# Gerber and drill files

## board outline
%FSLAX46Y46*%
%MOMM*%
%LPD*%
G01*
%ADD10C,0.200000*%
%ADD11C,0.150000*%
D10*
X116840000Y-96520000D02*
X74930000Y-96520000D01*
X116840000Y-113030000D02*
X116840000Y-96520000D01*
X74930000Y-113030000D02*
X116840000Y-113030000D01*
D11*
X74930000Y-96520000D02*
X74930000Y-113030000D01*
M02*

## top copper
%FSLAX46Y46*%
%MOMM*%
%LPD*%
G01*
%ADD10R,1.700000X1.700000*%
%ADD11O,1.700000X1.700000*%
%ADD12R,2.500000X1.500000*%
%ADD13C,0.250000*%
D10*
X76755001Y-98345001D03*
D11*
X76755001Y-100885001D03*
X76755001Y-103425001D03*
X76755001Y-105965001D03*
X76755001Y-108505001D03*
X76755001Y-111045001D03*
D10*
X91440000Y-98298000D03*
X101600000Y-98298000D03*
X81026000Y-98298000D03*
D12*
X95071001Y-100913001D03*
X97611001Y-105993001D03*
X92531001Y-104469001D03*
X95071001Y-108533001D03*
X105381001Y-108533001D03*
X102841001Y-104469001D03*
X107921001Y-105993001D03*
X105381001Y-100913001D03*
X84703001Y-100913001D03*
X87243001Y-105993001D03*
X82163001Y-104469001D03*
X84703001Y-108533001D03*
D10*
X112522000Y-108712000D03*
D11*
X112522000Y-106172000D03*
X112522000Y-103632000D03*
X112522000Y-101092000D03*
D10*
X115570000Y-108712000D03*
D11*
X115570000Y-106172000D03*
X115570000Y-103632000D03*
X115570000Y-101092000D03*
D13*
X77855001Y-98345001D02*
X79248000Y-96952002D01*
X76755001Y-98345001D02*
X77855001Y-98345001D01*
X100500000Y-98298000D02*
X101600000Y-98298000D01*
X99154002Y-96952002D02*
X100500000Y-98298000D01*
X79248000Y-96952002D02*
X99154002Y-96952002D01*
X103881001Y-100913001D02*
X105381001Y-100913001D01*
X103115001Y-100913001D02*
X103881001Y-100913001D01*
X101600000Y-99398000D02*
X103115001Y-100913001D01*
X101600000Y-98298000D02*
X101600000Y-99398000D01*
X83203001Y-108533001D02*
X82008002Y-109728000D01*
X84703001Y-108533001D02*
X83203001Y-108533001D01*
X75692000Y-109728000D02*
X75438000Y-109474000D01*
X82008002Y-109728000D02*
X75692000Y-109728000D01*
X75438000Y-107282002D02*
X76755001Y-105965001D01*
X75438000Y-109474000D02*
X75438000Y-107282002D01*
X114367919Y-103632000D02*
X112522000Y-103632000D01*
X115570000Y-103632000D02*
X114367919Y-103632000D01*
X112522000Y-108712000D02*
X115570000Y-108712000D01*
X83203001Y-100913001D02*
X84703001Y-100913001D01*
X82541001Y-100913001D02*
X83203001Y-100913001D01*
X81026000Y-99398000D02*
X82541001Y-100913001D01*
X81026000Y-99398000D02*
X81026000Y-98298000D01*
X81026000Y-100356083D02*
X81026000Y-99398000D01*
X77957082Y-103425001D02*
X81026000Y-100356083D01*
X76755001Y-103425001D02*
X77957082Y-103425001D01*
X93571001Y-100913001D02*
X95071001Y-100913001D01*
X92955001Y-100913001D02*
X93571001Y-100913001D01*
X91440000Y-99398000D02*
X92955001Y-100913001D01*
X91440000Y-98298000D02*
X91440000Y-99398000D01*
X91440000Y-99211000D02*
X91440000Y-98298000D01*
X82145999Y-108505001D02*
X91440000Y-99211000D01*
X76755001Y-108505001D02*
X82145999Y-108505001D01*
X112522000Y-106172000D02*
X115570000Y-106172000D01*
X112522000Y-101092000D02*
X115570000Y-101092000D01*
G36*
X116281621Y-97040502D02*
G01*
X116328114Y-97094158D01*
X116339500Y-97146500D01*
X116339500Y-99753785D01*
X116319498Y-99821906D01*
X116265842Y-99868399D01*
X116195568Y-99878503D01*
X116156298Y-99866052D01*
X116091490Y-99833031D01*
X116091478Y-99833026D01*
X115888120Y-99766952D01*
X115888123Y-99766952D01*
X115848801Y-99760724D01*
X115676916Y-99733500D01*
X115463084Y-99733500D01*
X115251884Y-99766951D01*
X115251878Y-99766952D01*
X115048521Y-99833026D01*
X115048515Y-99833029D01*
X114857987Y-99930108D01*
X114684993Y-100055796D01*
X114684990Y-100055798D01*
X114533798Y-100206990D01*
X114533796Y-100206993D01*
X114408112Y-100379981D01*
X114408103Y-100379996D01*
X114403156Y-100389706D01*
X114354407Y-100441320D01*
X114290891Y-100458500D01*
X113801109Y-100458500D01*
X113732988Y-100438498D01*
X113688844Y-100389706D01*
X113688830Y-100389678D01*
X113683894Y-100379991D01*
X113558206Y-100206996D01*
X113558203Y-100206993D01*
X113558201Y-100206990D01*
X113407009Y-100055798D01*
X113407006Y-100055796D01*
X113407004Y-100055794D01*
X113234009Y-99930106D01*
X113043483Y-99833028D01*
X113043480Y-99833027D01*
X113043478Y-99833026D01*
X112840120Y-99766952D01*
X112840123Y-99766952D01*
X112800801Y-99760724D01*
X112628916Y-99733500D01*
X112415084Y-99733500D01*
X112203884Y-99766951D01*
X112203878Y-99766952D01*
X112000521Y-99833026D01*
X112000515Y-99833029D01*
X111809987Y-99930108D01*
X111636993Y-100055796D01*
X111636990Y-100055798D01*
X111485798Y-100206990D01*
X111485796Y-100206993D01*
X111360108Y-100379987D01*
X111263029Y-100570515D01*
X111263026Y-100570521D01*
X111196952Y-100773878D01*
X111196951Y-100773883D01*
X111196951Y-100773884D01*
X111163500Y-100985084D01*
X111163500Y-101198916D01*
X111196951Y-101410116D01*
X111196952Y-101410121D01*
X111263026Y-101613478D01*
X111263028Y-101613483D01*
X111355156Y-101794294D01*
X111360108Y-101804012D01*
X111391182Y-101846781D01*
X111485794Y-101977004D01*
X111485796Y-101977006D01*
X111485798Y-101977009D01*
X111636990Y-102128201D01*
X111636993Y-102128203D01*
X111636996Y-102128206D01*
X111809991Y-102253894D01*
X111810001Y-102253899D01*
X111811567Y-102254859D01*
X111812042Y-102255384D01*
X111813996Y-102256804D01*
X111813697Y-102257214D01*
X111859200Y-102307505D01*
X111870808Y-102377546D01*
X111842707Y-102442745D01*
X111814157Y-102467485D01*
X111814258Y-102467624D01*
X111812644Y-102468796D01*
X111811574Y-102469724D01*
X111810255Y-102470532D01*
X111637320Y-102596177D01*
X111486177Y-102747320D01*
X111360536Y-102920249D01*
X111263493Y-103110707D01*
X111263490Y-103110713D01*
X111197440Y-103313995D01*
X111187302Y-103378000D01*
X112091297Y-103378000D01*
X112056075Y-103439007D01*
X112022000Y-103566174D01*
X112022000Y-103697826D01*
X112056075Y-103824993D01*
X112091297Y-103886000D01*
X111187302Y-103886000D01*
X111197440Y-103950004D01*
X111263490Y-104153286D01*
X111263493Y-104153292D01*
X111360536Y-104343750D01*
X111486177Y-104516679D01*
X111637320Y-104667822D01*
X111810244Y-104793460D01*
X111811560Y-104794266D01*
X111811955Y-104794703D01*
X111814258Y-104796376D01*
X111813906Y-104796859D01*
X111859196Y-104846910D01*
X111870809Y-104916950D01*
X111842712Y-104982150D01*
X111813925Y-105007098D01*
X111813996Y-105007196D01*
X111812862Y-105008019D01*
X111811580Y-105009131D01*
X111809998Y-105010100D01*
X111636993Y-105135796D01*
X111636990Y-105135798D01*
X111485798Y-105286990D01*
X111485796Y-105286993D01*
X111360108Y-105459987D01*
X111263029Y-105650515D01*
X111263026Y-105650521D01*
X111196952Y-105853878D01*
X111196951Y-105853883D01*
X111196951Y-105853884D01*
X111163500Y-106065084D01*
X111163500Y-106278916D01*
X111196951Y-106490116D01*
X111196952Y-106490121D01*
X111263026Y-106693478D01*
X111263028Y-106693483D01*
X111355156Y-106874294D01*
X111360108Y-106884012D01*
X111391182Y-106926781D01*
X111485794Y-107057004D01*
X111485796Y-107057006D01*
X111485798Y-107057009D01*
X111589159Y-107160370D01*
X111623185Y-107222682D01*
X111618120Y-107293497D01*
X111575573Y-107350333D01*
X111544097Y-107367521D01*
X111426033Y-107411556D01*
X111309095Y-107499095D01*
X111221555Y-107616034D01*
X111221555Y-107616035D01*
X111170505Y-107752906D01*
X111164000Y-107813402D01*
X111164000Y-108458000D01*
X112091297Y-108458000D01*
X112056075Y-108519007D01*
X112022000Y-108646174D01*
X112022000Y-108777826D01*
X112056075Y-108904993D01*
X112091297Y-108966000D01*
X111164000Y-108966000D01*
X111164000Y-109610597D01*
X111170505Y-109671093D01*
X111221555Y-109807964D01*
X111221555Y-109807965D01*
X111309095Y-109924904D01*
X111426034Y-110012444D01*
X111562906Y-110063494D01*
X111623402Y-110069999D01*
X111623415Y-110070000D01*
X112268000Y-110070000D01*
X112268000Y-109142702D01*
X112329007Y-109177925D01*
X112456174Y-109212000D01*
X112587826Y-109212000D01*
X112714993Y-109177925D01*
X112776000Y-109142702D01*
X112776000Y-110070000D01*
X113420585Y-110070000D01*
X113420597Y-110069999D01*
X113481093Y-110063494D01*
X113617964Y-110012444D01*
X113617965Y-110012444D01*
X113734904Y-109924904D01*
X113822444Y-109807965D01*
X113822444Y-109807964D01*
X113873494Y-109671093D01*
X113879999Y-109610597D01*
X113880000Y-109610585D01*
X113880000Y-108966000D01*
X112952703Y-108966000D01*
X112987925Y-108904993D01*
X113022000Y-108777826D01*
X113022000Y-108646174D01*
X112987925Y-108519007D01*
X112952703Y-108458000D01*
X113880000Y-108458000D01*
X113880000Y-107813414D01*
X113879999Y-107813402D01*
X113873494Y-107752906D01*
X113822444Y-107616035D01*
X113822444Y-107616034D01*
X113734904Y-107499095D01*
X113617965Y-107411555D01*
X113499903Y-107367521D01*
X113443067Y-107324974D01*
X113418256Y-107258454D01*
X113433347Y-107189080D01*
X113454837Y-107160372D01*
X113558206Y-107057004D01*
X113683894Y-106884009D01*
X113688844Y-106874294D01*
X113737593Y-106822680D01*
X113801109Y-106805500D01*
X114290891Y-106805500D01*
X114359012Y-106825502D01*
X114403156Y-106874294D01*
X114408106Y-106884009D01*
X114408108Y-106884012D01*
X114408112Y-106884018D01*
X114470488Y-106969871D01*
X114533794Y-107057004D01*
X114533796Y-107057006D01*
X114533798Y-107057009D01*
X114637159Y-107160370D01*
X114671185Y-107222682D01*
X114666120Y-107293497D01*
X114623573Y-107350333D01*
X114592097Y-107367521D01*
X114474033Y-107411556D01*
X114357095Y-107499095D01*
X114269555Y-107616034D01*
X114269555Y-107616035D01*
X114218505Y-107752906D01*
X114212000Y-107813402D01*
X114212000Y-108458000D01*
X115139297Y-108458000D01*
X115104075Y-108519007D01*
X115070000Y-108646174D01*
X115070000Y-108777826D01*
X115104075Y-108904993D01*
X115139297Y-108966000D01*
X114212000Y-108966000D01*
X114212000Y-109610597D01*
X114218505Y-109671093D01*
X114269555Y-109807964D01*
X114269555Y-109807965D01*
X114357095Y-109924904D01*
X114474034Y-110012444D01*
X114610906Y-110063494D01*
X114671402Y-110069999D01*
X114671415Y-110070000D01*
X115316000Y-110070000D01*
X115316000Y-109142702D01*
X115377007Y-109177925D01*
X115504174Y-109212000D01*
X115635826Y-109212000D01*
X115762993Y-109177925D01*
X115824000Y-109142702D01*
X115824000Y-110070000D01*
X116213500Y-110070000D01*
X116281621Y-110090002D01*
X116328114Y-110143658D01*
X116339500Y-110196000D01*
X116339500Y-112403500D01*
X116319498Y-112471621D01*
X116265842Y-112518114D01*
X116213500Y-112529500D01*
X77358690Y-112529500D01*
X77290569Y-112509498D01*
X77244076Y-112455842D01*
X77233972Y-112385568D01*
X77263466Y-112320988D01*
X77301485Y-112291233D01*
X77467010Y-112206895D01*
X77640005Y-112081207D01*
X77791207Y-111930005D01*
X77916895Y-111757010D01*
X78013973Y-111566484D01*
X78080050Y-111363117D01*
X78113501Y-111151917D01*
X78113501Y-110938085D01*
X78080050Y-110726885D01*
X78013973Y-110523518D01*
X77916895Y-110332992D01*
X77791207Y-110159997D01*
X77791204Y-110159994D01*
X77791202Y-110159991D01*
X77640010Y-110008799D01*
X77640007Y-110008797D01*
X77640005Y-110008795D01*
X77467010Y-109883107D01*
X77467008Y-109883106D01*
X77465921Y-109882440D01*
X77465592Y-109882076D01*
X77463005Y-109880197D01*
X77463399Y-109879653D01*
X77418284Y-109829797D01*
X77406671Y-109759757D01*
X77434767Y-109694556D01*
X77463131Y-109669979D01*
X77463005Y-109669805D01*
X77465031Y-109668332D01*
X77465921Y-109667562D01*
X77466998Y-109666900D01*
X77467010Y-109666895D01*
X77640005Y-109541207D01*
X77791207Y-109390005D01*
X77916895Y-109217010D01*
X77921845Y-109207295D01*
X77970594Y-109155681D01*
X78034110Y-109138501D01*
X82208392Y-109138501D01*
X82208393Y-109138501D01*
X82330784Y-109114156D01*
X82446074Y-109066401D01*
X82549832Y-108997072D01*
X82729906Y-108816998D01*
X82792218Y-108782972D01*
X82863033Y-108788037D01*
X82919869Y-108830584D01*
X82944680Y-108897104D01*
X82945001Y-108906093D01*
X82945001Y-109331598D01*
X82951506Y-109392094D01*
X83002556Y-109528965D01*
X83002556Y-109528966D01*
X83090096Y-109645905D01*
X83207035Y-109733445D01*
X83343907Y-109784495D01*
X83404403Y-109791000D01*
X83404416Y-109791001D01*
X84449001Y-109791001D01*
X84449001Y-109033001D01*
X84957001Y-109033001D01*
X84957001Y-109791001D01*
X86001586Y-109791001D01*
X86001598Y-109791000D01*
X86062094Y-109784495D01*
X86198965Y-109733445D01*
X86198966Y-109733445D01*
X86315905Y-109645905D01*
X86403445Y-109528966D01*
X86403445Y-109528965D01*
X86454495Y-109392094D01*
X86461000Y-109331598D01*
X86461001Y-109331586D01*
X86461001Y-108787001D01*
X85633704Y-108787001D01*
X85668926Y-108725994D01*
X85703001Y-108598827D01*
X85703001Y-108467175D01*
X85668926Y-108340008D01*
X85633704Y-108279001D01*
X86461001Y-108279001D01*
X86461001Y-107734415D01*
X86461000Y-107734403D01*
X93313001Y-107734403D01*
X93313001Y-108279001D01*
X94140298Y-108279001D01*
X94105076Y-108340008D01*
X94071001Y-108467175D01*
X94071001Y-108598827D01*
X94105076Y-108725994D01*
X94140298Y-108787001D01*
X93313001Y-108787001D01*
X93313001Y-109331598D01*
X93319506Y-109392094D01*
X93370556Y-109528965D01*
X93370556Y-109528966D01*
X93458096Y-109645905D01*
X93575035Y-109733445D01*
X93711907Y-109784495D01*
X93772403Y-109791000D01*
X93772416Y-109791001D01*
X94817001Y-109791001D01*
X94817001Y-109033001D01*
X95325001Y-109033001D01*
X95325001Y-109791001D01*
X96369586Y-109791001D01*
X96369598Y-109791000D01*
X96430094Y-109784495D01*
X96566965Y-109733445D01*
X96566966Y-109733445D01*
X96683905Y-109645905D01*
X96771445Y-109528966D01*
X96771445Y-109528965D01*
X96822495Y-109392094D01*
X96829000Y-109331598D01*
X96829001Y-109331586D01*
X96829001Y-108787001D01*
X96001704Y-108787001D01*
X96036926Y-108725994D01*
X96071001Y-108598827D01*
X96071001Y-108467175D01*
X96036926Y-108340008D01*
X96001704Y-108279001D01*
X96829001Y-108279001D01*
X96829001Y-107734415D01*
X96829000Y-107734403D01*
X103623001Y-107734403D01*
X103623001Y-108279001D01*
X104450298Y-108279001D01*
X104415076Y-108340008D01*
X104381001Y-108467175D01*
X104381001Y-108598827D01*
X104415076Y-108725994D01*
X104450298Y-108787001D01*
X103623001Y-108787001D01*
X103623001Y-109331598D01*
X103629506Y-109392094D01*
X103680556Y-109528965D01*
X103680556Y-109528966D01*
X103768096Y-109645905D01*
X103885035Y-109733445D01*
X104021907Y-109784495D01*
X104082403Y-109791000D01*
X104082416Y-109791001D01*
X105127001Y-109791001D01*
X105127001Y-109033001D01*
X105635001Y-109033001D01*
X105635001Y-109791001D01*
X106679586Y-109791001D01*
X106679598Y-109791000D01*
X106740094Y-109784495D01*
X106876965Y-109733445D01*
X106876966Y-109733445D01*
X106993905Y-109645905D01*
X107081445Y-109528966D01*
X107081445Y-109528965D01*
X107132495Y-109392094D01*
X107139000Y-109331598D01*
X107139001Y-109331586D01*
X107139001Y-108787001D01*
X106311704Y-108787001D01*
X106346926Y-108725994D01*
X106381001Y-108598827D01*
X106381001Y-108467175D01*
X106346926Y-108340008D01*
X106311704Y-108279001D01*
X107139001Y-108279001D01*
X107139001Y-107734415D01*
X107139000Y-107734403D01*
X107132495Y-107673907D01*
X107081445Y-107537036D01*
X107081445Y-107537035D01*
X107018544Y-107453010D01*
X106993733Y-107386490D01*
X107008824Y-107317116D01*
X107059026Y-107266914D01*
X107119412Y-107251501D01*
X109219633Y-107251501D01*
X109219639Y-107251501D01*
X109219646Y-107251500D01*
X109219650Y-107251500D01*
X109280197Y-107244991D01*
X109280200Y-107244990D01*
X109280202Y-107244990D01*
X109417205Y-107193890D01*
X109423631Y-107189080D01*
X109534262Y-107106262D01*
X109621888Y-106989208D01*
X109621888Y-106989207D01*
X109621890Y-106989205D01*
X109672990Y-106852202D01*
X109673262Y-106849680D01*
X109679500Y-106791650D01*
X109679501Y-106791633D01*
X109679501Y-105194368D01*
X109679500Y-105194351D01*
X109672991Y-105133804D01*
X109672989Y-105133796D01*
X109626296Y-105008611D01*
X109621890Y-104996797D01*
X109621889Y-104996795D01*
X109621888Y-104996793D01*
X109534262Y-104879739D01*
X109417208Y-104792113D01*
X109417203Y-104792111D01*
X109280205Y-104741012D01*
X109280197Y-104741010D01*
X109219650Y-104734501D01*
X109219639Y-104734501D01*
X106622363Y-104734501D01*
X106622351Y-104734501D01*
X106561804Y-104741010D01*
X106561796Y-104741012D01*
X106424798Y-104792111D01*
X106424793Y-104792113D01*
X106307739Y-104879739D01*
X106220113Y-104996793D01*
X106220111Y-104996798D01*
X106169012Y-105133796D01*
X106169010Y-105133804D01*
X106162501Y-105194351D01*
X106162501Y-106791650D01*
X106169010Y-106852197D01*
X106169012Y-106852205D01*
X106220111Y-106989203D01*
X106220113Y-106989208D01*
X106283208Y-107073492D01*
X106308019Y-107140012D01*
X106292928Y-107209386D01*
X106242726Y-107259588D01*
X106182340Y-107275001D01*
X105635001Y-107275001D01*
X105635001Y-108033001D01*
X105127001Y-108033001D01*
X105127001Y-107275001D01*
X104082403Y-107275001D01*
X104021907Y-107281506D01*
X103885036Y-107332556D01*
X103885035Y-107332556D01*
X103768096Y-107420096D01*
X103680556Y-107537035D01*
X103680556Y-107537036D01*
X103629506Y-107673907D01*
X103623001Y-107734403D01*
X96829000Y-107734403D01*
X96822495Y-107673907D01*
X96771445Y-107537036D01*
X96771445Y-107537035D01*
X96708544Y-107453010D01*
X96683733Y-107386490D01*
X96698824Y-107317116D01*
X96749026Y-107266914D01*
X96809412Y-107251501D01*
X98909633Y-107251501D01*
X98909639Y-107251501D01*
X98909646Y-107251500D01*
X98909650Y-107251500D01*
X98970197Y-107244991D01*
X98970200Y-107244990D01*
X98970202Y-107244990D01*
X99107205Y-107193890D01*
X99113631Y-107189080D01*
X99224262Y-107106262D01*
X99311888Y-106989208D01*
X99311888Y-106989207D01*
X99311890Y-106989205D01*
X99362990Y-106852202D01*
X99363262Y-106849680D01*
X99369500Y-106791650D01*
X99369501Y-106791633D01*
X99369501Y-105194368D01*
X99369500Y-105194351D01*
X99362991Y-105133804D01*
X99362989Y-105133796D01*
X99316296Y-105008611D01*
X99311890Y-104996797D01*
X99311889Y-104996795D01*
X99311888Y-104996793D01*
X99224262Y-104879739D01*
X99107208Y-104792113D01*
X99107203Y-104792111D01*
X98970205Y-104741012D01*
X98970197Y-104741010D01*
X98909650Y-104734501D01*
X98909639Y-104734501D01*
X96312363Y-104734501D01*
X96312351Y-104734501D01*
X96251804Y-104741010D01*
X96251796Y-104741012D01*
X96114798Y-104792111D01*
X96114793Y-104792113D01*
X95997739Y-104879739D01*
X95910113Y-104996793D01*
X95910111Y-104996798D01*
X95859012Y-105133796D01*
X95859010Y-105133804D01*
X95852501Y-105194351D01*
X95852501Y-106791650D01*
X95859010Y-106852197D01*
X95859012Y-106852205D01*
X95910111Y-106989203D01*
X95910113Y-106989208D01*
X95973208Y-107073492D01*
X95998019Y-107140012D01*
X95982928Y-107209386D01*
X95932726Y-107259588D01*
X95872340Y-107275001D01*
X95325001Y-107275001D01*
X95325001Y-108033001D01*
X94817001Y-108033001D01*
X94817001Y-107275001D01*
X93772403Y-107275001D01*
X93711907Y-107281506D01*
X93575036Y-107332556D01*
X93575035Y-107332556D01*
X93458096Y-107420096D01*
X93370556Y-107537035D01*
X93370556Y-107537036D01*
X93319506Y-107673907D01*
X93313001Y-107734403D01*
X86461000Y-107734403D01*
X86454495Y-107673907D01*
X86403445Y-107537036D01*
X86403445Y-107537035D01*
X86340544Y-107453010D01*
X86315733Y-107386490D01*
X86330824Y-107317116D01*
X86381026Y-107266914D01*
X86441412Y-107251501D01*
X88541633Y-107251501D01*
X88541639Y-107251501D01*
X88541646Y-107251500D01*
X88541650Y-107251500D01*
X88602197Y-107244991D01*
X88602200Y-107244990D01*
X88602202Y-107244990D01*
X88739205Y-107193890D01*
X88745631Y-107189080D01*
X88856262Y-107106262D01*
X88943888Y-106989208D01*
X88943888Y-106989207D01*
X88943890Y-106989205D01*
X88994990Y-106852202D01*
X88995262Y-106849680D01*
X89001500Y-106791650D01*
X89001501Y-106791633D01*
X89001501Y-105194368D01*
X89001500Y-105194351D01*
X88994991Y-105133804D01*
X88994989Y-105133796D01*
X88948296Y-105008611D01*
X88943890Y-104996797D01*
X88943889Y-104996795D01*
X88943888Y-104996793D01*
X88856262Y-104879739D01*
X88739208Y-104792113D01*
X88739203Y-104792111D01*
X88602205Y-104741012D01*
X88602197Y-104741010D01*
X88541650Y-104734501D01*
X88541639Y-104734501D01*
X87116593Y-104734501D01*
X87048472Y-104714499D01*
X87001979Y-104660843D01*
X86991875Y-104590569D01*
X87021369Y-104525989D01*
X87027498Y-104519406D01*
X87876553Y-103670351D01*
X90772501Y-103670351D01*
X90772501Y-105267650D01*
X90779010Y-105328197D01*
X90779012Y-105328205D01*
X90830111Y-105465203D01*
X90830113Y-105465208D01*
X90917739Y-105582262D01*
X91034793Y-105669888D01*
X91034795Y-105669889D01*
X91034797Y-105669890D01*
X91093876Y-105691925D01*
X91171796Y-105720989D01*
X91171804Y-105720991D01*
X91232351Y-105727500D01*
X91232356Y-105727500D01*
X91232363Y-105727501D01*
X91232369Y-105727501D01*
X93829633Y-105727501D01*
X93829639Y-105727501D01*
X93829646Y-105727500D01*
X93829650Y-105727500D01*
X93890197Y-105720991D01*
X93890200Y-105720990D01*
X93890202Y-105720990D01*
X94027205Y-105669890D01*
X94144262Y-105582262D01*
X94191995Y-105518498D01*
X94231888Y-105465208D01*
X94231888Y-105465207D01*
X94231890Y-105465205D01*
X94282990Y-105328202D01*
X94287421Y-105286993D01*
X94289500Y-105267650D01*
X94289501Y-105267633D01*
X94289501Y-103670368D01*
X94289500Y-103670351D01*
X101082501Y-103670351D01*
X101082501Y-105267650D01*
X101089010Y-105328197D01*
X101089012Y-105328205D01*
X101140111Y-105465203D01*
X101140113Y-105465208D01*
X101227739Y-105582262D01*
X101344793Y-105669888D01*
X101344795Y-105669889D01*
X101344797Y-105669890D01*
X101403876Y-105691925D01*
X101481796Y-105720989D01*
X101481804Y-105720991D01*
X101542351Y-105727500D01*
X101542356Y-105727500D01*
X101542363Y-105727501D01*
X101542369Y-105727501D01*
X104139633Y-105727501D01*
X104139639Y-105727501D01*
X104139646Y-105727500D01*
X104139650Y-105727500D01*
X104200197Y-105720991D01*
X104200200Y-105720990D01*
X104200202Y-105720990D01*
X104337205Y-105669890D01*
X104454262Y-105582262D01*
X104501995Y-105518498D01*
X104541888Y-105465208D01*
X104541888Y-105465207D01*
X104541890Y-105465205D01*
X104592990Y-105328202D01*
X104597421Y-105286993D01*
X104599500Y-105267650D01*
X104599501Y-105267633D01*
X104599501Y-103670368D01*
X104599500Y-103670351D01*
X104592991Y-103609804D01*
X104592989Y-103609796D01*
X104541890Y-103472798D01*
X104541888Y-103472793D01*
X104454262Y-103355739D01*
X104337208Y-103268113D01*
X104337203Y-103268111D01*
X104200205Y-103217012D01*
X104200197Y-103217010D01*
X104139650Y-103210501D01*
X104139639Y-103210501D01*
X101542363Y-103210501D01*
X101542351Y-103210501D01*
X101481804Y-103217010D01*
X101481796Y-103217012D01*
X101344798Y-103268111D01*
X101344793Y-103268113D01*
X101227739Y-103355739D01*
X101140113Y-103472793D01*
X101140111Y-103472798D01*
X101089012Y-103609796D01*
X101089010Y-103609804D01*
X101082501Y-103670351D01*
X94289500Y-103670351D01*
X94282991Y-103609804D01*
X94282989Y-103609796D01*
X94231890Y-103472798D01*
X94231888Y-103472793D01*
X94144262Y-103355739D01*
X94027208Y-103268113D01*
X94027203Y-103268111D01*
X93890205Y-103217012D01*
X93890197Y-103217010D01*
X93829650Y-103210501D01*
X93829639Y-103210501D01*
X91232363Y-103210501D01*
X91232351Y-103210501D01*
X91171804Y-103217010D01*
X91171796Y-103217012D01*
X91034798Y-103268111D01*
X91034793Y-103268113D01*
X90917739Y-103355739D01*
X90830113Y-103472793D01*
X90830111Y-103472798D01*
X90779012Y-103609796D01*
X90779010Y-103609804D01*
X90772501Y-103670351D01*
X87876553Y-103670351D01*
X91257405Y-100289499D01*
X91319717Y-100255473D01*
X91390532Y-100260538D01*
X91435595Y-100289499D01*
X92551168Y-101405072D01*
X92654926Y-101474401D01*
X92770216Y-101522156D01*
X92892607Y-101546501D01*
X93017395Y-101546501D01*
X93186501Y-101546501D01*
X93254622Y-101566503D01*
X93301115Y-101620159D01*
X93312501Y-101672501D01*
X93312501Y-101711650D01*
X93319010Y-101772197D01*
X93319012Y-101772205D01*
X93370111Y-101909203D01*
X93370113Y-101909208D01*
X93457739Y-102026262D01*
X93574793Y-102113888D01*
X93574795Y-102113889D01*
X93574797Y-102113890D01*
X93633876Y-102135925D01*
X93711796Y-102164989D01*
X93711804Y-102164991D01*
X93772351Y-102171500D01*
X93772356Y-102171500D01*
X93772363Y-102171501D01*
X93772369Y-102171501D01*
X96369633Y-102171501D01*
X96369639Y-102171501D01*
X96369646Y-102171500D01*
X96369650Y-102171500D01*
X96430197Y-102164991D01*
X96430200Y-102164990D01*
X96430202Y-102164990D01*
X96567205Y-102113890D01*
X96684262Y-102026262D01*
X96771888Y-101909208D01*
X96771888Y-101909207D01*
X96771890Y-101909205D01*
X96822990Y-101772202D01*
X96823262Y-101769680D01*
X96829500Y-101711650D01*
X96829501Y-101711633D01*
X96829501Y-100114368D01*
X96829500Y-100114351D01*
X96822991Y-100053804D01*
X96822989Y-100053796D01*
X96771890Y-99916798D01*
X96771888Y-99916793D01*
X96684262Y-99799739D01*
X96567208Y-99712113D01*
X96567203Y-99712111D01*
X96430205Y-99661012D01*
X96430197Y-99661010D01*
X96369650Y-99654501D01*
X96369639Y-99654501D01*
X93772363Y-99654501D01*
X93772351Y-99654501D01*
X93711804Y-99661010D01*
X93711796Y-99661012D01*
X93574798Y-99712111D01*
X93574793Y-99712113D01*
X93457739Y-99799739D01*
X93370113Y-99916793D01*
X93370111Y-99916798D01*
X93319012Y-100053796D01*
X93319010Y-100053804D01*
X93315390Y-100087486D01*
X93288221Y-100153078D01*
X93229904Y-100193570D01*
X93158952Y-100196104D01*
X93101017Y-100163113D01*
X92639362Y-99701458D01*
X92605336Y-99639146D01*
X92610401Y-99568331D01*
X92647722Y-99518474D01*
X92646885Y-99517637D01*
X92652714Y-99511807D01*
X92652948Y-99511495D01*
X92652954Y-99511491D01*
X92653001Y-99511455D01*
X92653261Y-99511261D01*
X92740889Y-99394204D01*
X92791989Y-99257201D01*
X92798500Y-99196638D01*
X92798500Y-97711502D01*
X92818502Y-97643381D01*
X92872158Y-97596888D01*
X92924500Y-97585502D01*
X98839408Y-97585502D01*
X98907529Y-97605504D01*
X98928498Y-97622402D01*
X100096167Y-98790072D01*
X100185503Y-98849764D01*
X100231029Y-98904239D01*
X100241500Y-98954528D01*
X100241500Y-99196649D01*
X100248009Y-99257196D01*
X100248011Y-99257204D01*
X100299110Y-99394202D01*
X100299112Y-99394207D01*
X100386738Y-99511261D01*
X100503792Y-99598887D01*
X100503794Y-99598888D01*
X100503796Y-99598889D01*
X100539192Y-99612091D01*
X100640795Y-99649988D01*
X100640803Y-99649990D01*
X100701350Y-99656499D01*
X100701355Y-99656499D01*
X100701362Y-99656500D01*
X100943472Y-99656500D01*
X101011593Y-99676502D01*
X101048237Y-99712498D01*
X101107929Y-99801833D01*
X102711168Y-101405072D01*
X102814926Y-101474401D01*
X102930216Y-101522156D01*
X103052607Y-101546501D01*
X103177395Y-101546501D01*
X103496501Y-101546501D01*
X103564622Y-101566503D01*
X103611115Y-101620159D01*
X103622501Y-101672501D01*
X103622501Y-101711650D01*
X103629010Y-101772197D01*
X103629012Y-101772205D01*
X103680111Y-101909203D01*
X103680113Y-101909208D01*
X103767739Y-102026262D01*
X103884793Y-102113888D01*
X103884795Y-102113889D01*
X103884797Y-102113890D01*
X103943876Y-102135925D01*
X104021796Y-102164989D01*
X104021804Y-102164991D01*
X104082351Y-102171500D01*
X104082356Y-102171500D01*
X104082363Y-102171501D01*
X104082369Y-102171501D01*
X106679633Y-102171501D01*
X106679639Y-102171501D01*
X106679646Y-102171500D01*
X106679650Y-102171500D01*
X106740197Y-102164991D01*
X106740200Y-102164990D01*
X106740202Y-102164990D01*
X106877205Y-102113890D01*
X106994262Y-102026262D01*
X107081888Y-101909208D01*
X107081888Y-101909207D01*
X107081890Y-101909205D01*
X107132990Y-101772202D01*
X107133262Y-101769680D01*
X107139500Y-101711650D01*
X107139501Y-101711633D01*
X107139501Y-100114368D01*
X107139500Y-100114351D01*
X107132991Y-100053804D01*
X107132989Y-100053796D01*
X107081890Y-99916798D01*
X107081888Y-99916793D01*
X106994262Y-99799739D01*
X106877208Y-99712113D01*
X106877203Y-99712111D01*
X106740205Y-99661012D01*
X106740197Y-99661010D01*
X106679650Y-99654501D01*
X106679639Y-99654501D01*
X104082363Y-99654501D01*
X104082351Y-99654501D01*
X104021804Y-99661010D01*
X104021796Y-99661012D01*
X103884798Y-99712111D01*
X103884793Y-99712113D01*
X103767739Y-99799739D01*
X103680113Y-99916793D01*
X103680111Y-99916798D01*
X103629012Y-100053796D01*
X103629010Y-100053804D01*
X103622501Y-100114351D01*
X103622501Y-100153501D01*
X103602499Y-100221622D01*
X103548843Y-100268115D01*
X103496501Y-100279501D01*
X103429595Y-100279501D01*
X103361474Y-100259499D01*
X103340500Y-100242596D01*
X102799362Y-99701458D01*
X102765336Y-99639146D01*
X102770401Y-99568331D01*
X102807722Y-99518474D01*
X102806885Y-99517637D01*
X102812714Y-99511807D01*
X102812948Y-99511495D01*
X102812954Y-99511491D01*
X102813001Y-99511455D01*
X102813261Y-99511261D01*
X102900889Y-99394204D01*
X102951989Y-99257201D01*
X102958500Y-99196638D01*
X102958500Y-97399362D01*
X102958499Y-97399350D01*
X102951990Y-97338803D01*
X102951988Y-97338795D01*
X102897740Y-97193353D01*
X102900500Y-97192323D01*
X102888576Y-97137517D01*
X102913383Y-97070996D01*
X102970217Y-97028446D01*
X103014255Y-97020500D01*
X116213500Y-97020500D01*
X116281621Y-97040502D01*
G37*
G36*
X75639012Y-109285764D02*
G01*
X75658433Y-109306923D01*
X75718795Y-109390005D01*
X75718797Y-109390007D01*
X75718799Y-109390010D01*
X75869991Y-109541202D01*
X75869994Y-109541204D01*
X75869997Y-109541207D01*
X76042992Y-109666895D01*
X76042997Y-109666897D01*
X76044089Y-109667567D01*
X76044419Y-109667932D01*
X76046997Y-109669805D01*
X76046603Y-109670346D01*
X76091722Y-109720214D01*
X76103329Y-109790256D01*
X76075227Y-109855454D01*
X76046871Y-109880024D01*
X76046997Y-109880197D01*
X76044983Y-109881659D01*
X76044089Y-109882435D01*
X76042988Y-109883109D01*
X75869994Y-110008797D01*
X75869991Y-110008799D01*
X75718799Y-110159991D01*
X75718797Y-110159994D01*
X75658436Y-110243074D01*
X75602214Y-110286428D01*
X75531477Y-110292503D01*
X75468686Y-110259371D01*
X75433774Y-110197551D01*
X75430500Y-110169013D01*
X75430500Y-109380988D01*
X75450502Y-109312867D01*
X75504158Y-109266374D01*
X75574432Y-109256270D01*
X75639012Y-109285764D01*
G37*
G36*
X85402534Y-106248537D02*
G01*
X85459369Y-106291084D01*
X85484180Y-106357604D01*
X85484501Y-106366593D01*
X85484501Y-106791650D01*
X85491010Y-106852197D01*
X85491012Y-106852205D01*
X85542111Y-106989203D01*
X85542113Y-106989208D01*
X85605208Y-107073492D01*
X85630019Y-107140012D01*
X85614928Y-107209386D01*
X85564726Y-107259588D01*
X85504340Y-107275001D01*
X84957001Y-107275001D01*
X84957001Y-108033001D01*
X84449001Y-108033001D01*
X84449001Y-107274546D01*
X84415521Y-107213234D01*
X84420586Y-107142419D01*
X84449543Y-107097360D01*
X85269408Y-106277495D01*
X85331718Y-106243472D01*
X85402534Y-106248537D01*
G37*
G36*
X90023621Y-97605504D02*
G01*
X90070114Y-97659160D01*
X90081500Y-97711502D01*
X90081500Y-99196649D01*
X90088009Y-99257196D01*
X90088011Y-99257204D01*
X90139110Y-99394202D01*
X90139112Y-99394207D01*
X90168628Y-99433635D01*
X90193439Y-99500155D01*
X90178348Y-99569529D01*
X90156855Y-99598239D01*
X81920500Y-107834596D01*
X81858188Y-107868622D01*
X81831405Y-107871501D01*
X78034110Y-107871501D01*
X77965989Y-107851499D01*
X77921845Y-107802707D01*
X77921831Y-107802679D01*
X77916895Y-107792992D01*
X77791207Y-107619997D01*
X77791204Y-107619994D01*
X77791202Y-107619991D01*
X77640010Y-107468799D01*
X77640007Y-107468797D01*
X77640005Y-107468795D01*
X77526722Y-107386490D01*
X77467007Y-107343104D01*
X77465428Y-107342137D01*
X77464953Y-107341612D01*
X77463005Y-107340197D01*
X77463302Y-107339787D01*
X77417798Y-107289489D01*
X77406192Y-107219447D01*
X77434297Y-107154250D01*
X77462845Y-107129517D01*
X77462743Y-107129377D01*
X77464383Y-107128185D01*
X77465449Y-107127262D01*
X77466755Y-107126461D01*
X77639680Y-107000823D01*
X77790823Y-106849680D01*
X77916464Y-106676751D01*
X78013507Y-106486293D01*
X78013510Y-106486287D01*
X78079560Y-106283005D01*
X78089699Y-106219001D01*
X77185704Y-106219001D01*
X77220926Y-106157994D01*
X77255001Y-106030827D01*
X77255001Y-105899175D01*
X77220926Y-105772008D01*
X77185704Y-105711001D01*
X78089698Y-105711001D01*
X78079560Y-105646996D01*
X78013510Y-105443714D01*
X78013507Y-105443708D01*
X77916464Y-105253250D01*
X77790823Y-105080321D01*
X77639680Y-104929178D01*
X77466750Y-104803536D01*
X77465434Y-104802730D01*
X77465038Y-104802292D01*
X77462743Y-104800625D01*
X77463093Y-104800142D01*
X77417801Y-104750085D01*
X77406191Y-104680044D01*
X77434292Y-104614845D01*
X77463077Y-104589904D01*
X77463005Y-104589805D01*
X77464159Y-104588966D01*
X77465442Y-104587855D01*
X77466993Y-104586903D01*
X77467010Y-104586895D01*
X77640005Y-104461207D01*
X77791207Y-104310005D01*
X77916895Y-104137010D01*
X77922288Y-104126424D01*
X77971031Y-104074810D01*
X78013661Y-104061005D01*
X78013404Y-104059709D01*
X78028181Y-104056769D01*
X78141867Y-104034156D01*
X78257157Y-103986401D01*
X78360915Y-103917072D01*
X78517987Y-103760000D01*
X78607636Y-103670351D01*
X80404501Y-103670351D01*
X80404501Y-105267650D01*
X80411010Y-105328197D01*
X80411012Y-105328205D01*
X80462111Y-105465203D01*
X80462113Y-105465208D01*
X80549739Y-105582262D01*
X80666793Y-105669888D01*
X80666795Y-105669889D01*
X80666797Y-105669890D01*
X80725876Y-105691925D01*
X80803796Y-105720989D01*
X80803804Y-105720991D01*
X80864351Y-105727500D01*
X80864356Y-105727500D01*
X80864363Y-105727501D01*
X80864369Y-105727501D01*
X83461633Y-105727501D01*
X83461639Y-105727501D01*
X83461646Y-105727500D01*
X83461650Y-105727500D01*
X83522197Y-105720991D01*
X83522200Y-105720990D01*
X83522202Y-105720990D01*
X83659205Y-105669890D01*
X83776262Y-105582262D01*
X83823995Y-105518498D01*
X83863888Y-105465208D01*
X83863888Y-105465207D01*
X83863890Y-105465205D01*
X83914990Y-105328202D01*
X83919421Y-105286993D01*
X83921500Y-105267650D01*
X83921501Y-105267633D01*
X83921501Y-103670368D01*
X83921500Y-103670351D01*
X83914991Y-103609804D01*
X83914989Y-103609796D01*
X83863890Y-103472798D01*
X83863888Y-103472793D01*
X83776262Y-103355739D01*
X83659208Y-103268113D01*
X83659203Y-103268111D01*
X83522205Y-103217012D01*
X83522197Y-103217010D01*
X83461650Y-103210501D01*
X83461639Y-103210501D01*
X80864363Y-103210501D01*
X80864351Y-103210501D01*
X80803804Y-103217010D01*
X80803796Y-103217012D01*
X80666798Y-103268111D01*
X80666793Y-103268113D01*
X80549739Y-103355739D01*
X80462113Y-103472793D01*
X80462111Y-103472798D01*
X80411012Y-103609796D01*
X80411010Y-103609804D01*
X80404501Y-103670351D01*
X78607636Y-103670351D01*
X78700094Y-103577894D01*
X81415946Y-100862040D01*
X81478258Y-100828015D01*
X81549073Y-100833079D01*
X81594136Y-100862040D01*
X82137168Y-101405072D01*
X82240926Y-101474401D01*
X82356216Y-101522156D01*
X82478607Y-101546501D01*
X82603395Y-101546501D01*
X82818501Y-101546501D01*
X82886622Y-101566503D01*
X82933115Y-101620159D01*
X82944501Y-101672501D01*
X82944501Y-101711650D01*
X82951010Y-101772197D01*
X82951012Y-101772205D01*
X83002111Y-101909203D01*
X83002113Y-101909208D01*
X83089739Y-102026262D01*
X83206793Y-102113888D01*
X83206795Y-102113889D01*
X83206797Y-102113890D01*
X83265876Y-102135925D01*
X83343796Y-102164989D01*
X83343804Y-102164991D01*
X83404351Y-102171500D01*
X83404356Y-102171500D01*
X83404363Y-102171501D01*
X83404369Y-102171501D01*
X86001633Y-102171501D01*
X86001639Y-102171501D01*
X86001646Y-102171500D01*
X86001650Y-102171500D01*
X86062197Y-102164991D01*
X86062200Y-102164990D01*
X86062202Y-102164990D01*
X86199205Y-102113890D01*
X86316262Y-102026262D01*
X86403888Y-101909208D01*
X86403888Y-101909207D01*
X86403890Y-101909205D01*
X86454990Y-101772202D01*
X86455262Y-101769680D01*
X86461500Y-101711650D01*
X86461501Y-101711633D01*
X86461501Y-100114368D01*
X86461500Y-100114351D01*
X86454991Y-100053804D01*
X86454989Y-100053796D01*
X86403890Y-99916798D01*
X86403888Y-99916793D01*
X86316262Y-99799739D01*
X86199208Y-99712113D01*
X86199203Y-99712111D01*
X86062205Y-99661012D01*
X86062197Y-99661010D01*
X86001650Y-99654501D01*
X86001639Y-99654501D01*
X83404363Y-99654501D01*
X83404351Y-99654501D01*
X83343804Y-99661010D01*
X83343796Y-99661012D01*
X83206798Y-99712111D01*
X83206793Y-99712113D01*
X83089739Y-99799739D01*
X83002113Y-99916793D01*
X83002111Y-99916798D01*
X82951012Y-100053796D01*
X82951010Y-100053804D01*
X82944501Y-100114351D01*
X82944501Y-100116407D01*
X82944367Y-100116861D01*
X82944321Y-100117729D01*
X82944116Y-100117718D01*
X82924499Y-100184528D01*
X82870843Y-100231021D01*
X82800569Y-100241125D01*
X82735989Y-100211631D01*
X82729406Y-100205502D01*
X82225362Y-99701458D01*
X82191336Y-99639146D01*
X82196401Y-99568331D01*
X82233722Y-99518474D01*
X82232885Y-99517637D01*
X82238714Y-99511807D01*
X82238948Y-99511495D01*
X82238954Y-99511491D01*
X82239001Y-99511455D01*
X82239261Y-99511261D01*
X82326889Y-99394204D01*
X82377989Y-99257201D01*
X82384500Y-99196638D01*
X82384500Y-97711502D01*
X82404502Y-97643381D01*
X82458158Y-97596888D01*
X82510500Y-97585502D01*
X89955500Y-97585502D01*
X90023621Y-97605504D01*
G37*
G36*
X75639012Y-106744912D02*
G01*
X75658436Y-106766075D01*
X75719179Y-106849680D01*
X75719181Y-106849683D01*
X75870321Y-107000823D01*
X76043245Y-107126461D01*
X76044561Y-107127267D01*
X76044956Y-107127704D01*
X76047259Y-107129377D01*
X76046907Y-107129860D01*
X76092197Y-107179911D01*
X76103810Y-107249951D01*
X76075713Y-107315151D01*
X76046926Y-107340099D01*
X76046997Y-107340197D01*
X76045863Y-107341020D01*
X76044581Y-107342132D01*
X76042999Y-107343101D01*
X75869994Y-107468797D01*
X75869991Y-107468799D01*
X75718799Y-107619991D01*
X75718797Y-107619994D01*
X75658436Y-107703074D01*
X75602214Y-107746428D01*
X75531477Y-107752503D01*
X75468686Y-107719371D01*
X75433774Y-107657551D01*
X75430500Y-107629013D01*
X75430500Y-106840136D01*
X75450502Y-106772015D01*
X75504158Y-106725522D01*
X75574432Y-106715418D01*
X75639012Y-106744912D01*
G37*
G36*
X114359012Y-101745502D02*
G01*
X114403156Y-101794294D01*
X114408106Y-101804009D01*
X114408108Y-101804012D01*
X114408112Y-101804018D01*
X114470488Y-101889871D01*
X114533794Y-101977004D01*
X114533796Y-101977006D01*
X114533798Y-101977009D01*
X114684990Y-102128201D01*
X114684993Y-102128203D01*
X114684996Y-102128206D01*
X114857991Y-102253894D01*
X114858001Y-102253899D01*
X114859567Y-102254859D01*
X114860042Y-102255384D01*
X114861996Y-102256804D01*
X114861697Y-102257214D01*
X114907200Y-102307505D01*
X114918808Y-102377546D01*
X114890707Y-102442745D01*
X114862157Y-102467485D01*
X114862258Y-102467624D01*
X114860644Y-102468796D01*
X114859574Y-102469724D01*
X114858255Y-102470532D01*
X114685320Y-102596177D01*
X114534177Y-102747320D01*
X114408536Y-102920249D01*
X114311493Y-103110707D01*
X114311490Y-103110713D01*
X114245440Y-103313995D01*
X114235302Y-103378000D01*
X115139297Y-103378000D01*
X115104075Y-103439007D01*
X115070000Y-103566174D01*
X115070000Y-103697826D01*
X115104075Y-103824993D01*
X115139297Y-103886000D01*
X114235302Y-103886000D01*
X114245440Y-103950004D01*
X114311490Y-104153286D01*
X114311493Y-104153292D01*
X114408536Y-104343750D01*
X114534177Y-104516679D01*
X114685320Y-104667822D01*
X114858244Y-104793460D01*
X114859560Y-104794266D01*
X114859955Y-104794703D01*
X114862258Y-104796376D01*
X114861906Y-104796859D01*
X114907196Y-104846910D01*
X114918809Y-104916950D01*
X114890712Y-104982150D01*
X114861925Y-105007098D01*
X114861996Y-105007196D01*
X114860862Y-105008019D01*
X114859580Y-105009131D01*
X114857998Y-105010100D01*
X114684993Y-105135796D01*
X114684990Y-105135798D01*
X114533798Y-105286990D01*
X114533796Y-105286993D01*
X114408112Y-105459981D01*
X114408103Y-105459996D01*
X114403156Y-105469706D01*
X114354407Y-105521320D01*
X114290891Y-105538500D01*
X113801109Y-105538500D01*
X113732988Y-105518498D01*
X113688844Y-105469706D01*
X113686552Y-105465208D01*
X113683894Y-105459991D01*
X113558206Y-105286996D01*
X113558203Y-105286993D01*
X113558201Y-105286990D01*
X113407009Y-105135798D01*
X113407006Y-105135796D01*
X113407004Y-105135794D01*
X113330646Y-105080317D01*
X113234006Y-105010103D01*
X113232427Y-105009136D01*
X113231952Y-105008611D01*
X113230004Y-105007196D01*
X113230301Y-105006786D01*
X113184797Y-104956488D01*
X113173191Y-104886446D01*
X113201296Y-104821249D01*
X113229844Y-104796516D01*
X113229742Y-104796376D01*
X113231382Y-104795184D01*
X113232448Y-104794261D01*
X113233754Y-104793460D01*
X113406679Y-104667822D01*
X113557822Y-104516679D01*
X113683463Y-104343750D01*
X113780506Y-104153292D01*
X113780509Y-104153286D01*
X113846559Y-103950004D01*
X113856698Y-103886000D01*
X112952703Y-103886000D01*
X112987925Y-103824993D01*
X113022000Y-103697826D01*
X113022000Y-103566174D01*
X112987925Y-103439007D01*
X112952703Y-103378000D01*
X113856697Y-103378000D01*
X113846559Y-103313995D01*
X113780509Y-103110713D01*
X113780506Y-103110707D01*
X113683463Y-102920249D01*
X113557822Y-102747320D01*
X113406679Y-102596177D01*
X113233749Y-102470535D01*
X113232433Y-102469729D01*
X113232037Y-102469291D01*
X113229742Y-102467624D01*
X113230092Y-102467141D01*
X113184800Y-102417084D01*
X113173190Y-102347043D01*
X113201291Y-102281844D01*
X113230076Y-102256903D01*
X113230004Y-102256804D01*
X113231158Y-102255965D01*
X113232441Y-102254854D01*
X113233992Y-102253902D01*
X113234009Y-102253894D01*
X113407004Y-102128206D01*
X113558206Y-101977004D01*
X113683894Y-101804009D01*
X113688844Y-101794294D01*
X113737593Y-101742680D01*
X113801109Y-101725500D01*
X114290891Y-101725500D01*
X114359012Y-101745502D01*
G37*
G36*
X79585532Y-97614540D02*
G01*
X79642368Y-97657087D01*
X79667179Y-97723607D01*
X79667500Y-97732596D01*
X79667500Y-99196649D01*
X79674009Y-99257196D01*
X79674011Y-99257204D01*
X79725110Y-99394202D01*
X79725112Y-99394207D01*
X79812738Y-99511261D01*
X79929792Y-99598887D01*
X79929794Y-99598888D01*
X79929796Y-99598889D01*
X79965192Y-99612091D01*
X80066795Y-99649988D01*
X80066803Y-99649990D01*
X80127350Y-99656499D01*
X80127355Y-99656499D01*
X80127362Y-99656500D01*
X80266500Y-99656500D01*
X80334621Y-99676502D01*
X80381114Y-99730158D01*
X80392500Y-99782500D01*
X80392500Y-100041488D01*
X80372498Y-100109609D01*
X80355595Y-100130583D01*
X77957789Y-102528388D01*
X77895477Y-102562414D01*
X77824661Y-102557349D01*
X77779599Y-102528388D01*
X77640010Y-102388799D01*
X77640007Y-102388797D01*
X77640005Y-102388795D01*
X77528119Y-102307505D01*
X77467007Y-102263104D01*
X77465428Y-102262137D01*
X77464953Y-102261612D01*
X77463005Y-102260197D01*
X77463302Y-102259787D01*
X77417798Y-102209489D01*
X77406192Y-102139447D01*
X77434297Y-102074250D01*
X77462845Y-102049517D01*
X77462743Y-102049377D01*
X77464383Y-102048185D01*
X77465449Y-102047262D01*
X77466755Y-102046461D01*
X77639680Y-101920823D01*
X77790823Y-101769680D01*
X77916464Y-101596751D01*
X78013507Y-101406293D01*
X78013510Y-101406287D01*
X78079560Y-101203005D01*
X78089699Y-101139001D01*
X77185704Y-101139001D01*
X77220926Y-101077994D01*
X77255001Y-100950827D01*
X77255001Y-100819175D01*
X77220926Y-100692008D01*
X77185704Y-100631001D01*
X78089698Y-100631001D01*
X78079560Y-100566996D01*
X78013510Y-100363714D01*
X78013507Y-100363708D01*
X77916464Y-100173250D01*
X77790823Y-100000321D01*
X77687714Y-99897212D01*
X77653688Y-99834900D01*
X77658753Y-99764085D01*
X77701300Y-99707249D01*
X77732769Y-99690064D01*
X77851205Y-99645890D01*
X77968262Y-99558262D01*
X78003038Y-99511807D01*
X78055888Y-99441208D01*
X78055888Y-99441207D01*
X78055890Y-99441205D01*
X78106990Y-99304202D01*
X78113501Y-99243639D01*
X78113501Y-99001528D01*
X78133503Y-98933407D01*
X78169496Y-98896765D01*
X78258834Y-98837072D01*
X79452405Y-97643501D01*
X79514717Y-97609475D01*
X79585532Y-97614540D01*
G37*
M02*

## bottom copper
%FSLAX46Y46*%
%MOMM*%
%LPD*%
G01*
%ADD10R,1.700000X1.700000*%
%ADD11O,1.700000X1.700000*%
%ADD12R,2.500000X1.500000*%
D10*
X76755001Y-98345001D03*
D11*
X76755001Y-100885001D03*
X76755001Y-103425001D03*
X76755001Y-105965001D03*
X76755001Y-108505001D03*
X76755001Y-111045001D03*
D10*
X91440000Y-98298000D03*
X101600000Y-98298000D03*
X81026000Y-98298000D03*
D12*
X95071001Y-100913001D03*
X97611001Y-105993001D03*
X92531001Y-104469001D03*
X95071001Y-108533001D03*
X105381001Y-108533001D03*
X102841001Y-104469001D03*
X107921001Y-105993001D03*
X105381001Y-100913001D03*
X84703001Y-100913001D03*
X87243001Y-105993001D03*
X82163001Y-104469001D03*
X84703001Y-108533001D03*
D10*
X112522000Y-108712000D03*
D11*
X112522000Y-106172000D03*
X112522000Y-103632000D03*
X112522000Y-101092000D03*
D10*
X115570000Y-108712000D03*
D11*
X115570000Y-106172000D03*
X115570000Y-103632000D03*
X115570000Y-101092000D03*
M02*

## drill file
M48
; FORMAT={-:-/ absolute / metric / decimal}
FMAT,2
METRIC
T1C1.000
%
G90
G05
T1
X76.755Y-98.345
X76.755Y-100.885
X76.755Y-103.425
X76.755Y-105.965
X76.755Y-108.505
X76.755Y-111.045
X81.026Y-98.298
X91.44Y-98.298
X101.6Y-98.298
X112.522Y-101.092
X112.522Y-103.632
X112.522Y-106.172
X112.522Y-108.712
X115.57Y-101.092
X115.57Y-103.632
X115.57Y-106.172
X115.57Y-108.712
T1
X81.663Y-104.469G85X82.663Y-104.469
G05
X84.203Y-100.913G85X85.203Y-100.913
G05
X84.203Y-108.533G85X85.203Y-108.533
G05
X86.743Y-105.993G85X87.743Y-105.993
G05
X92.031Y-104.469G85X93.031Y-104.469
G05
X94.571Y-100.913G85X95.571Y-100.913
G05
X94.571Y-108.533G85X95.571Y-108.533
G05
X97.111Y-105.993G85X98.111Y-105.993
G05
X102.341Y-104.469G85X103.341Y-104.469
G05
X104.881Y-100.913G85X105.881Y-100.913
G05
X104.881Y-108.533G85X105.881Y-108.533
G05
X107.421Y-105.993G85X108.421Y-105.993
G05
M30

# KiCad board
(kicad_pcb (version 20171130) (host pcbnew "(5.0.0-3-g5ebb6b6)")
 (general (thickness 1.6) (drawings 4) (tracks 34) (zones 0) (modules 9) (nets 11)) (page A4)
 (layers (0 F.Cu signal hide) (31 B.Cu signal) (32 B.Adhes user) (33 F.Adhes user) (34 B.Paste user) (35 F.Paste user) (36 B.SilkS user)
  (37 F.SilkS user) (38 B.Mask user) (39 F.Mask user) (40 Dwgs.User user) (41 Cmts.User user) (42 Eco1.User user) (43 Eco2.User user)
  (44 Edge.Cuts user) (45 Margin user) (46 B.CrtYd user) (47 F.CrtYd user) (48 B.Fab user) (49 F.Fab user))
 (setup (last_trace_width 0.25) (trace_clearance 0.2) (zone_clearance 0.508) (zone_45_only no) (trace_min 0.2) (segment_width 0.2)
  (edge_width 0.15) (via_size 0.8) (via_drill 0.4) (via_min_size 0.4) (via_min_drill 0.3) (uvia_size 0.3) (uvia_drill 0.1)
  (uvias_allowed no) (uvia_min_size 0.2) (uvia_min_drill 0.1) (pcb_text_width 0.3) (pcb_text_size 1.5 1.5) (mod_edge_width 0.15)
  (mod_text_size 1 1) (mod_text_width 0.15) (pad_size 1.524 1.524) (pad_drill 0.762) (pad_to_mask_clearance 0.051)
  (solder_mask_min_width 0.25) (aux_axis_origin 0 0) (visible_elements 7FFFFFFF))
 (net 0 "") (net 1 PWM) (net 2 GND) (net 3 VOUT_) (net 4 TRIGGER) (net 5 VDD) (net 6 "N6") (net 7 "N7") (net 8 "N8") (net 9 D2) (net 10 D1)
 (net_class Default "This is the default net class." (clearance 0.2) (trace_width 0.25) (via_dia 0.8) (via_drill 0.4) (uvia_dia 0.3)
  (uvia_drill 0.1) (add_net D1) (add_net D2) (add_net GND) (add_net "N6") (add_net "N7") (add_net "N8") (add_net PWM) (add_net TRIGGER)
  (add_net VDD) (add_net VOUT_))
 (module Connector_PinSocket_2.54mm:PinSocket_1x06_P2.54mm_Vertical (layer F.Cu) (at 76.755001 98.345001)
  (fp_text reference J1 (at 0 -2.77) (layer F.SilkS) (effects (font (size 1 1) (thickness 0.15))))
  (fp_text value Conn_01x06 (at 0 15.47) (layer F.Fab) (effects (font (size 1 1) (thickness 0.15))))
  (pad 1 thru_hole rect (at 0 0) (size 1.7 1.7) (drill 1) (layers *.Cu *.Mask) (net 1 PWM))
  (pad 2 thru_hole oval (at 0 2.54) (size 1.7 1.7) (drill 1) (layers *.Cu *.Mask) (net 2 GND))
  (pad 3 thru_hole oval (at 0 5.08) (size 1.7 1.7) (drill 1) (layers *.Cu *.Mask) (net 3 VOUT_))
  (pad 4 thru_hole oval (at 0 7.62) (size 1.7 1.7) (drill 1) (layers *.Cu *.Mask) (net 2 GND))
  (pad 5 thru_hole oval (at 0 10.16) (size 1.7 1.7) (drill 1) (layers *.Cu *.Mask) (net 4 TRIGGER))
  (pad 6 thru_hole oval (at 0 12.7) (size 1.7 1.7) (drill 1) (layers *.Cu *.Mask) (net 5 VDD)))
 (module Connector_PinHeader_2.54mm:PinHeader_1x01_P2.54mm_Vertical (layer F.Cu) (at 91.44 98.298)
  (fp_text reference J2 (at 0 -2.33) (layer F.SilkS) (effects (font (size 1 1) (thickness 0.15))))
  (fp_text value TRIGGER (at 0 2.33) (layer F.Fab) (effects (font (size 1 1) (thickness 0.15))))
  (pad 1 thru_hole rect (at 0 0) (size 1.7 1.7) (drill 1) (layers *.Cu *.Mask) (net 4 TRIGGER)))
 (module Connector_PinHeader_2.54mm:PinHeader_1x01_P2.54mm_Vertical (layer F.Cu) (at 101.6 98.298)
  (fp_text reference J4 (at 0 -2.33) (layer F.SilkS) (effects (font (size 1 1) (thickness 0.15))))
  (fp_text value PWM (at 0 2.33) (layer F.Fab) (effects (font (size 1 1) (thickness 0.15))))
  (pad 1 thru_hole rect (at 0 0) (size 1.7 1.7) (drill 1) (layers *.Cu *.Mask) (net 1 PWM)))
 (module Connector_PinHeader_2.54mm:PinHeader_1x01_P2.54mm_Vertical (layer F.Cu) (at 81.026 98.298)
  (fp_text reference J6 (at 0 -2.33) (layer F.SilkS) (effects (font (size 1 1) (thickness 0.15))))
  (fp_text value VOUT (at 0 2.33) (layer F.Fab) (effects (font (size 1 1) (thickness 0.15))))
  (pad 1 thru_hole rect (at 0 0) (size 1.7 1.7) (drill 1) (layers *.Cu *.Mask) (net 3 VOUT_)))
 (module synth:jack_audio (layer F.Cu) (at 95.071001 105.993001)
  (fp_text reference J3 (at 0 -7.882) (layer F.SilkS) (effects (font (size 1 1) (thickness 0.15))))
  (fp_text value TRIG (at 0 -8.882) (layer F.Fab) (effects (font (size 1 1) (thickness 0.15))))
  (pad T thru_hole rect (at 0 -5.08) (size 2.5 1.5) (drill oval 2 1) (layers *.Cu *.Mask) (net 4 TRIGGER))
  (pad R thru_hole rect (at 2.54 0) (size 2.5 1.5) (drill oval 2 1) (layers *.Cu *.Mask) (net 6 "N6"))
  (pad GND thru_hole rect (at -2.54 -1.524) (size 2.5 1.5) (drill oval 2 1) (layers *.Cu *.Mask))
  (pad S thru_hole rect (at 0 2.54) (size 2.5 1.5) (drill oval 2 1) (layers *.Cu *.Mask) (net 2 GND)))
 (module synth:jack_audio (layer F.Cu) (at 105.381001 105.993001)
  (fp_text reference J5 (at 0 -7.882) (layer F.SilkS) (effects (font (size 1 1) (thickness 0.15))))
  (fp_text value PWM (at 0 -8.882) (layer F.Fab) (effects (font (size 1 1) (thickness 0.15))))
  (pad S thru_hole rect (at 0 2.54) (size 2.5 1.5) (drill oval 2 1) (layers *.Cu *.Mask) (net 2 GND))
  (pad GND thru_hole rect (at -2.54 -1.524) (size 2.5 1.5) (drill oval 2 1) (layers *.Cu *.Mask))
  (pad R thru_hole rect (at 2.54 0) (size 2.5 1.5) (drill oval 2 1) (layers *.Cu *.Mask) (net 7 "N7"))
  (pad T thru_hole rect (at 0 -5.08) (size 2.5 1.5) (drill oval 2 1) (layers *.Cu *.Mask) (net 1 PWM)))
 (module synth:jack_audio (layer F.Cu) (at 84.703001 105.993001)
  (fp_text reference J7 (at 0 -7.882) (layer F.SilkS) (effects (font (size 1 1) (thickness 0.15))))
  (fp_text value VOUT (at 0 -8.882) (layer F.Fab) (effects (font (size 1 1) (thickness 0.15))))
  (pad T thru_hole rect (at 0 -5.08) (size 2.5 1.5) (drill oval 2 1) (layers *.Cu *.Mask) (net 3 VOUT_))
  (pad R thru_hole rect (at 2.54 0) (size 2.5 1.5) (drill oval 2 1) (layers *.Cu *.Mask) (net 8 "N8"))
  (pad GND thru_hole rect (at -2.54 -1.524) (size 2.5 1.5) (drill oval 2 1) (layers *.Cu *.Mask))
  (pad S thru_hole rect (at 0 2.54) (size 2.5 1.5) (drill oval 2 1) (layers *.Cu *.Mask) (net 2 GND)))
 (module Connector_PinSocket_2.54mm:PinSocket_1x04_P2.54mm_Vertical (layer F.Cu) (at 112.522 108.712 180)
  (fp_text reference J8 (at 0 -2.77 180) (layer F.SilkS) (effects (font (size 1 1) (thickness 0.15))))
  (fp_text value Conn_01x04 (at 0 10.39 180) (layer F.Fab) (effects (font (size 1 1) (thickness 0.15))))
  (pad 1 thru_hole rect (at 0 0 180) (size 1.7 1.7) (drill 1) (layers *.Cu *.Mask) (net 2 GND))
  (pad 2 thru_hole oval (at 0 2.54 180) (size 1.7 1.7) (drill 1) (layers *.Cu *.Mask) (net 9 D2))
  (pad 3 thru_hole oval (at 0 5.08 180) (size 1.7 1.7) (drill 1) (layers *.Cu *.Mask) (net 2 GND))
  (pad 4 thru_hole oval (at 0 7.62 180) (size 1.7 1.7) (drill 1) (layers *.Cu *.Mask) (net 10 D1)))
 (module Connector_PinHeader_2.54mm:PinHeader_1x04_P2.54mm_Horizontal (layer B.Cu) (at 115.57 108.712)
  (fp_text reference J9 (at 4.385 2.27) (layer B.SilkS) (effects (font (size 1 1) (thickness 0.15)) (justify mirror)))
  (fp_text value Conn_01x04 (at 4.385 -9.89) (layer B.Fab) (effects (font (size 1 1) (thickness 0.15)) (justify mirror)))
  (pad 1 thru_hole rect (at 0 0) (size 1.7 1.7) (drill 1) (layers *.Cu *.Mask) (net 2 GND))
  (pad 2 thru_hole oval (at 0 -2.54) (size 1.7 1.7) (drill 1) (layers *.Cu *.Mask) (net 9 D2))
  (pad 3 thru_hole oval (at 0 -5.08) (size 1.7 1.7) (drill 1) (layers *.Cu *.Mask) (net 2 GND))
  (pad 4 thru_hole oval (at 0 -7.62) (size 1.7 1.7) (drill 1) (layers *.Cu *.Mask) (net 10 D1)))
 (gr_line (start 116.84 96.52) (end 74.93 96.52) (layer Edge.Cuts) (width 0.2))
 (gr_line (start 116.84 113.03) (end 116.84 96.52) (layer Edge.Cuts) (width 0.2))
 (gr_line (start 74.93 113.03) (end 116.84 113.03) (layer Edge.Cuts) (width 0.2))
 (gr_line (start 74.93 96.52) (end 74.93 113.03) (layer Edge.Cuts) (width 0.15))
 (segment (start 77.855001 98.345001) (end 79.248 96.952002) (width 0.25) (layer F.Cu) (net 1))
 (segment (start 76.755001 98.345001) (end 77.855001 98.345001) (width 0.25) (layer F.Cu) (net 1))
 (segment (start 100.5 98.298) (end 101.6 98.298) (width 0.25) (layer F.Cu) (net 1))
 (segment (start 99.154002 96.952002) (end 100.5 98.298) (width 0.25) (layer F.Cu) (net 1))
 (segment (start 79.248 96.952002) (end 99.154002 96.952002) (width 0.25) (layer F.Cu) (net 1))
 (segment (start 103.881001 100.913001) (end 105.381001 100.913001) (width 0.25) (layer F.Cu) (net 1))
 (segment (start 103.115001 100.913001) (end 103.881001 100.913001) (width 0.25) (layer F.Cu) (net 1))
 (segment (start 101.6 99.398) (end 103.115001 100.913001) (width 0.25) (layer F.Cu) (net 1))
 (segment (start 101.6 98.298) (end 101.6 99.398) (width 0.25) (layer F.Cu) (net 1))
 (segment (start 83.203001 108.533001) (end 82.008002 109.728) (width 0.25) (layer F.Cu) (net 2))
 (segment (start 84.703001 108.533001) (end 83.203001 108.533001) (width 0.25) (layer F.Cu) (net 2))
 (segment (start 75.692 109.728) (end 75.438 109.474) (width 0.25) (layer F.Cu) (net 2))
 (segment (start 82.008002 109.728) (end 75.692 109.728) (width 0.25) (layer F.Cu) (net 2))
 (segment (start 75.438 107.282002) (end 76.755001 105.965001) (width 0.25) (layer F.Cu) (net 2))
 (segment (start 75.438 109.474) (end 75.438 107.282002) (width 0.25) (layer F.Cu) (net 2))
 (segment (start 114.367919 103.632) (end 112.522 103.632) (width 0.25) (layer F.Cu) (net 2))
 (segment (start 115.57 103.632) (end 114.367919 103.632) (width 0.25) (layer F.Cu) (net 2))
 (segment (start 112.522 108.712) (end 115.57 108.712) (width 0.25) (layer F.Cu) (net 2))
 (segment (start 83.203001 100.913001) (end 84.703001 100.913001) (width 0.25) (layer F.Cu) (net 3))
 (segment (start 82.541001 100.913001) (end 83.203001 100.913001) (width 0.25) (layer F.Cu) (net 3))
 (segment (start 81.026 99.398) (end 82.541001 100.913001) (width 0.25) (layer F.Cu) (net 3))
 (segment (start 81.026 99.398) (end 81.026 98.298) (width 0.25) (layer F.Cu) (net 3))
 (segment (start 81.026 100.356083) (end 81.026 99.398) (width 0.25) (layer F.Cu) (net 3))
 (segment (start 77.957082 103.425001) (end 81.026 100.356083) (width 0.25) (layer F.Cu) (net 3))
 (segment (start 76.755001 103.425001) (end 77.957082 103.425001) (width 0.25) (layer F.Cu) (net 3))
 (segment (start 93.571001 100.913001) (end 95.071001 100.913001) (width 0.25) (layer F.Cu) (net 4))
 (segment (start 92.955001 100.913001) (end 93.571001 100.913001) (width 0.25) (layer F.Cu) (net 4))
 (segment (start 91.44 99.398) (end 92.955001 100.913001) (width 0.25) (layer F.Cu) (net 4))
 (segment (start 91.44 98.298) (end 91.44 99.398) (width 0.25) (layer F.Cu) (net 4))
 (segment (start 91.44 99.211) (end 91.44 98.298) (width 0.25) (layer F.Cu) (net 4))
 (segment (start 82.145999 108.505001) (end 91.44 99.211) (width 0.25) (layer F.Cu) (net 4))
 (segment (start 76.755001 108.505001) (end 82.145999 108.505001) (width 0.25) (layer F.Cu) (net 4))
 (segment (start 112.522 106.172) (end 115.57 106.172) (width 0.25) (layer F.Cu) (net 9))
 (segment (start 112.522 101.092) (end 115.57 101.092) (width 0.25) (layer F.Cu) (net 10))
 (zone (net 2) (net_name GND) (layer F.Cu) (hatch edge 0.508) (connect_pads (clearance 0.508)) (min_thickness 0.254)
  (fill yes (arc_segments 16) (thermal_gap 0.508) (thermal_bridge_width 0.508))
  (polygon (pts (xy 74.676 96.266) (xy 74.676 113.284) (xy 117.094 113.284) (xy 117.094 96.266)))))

